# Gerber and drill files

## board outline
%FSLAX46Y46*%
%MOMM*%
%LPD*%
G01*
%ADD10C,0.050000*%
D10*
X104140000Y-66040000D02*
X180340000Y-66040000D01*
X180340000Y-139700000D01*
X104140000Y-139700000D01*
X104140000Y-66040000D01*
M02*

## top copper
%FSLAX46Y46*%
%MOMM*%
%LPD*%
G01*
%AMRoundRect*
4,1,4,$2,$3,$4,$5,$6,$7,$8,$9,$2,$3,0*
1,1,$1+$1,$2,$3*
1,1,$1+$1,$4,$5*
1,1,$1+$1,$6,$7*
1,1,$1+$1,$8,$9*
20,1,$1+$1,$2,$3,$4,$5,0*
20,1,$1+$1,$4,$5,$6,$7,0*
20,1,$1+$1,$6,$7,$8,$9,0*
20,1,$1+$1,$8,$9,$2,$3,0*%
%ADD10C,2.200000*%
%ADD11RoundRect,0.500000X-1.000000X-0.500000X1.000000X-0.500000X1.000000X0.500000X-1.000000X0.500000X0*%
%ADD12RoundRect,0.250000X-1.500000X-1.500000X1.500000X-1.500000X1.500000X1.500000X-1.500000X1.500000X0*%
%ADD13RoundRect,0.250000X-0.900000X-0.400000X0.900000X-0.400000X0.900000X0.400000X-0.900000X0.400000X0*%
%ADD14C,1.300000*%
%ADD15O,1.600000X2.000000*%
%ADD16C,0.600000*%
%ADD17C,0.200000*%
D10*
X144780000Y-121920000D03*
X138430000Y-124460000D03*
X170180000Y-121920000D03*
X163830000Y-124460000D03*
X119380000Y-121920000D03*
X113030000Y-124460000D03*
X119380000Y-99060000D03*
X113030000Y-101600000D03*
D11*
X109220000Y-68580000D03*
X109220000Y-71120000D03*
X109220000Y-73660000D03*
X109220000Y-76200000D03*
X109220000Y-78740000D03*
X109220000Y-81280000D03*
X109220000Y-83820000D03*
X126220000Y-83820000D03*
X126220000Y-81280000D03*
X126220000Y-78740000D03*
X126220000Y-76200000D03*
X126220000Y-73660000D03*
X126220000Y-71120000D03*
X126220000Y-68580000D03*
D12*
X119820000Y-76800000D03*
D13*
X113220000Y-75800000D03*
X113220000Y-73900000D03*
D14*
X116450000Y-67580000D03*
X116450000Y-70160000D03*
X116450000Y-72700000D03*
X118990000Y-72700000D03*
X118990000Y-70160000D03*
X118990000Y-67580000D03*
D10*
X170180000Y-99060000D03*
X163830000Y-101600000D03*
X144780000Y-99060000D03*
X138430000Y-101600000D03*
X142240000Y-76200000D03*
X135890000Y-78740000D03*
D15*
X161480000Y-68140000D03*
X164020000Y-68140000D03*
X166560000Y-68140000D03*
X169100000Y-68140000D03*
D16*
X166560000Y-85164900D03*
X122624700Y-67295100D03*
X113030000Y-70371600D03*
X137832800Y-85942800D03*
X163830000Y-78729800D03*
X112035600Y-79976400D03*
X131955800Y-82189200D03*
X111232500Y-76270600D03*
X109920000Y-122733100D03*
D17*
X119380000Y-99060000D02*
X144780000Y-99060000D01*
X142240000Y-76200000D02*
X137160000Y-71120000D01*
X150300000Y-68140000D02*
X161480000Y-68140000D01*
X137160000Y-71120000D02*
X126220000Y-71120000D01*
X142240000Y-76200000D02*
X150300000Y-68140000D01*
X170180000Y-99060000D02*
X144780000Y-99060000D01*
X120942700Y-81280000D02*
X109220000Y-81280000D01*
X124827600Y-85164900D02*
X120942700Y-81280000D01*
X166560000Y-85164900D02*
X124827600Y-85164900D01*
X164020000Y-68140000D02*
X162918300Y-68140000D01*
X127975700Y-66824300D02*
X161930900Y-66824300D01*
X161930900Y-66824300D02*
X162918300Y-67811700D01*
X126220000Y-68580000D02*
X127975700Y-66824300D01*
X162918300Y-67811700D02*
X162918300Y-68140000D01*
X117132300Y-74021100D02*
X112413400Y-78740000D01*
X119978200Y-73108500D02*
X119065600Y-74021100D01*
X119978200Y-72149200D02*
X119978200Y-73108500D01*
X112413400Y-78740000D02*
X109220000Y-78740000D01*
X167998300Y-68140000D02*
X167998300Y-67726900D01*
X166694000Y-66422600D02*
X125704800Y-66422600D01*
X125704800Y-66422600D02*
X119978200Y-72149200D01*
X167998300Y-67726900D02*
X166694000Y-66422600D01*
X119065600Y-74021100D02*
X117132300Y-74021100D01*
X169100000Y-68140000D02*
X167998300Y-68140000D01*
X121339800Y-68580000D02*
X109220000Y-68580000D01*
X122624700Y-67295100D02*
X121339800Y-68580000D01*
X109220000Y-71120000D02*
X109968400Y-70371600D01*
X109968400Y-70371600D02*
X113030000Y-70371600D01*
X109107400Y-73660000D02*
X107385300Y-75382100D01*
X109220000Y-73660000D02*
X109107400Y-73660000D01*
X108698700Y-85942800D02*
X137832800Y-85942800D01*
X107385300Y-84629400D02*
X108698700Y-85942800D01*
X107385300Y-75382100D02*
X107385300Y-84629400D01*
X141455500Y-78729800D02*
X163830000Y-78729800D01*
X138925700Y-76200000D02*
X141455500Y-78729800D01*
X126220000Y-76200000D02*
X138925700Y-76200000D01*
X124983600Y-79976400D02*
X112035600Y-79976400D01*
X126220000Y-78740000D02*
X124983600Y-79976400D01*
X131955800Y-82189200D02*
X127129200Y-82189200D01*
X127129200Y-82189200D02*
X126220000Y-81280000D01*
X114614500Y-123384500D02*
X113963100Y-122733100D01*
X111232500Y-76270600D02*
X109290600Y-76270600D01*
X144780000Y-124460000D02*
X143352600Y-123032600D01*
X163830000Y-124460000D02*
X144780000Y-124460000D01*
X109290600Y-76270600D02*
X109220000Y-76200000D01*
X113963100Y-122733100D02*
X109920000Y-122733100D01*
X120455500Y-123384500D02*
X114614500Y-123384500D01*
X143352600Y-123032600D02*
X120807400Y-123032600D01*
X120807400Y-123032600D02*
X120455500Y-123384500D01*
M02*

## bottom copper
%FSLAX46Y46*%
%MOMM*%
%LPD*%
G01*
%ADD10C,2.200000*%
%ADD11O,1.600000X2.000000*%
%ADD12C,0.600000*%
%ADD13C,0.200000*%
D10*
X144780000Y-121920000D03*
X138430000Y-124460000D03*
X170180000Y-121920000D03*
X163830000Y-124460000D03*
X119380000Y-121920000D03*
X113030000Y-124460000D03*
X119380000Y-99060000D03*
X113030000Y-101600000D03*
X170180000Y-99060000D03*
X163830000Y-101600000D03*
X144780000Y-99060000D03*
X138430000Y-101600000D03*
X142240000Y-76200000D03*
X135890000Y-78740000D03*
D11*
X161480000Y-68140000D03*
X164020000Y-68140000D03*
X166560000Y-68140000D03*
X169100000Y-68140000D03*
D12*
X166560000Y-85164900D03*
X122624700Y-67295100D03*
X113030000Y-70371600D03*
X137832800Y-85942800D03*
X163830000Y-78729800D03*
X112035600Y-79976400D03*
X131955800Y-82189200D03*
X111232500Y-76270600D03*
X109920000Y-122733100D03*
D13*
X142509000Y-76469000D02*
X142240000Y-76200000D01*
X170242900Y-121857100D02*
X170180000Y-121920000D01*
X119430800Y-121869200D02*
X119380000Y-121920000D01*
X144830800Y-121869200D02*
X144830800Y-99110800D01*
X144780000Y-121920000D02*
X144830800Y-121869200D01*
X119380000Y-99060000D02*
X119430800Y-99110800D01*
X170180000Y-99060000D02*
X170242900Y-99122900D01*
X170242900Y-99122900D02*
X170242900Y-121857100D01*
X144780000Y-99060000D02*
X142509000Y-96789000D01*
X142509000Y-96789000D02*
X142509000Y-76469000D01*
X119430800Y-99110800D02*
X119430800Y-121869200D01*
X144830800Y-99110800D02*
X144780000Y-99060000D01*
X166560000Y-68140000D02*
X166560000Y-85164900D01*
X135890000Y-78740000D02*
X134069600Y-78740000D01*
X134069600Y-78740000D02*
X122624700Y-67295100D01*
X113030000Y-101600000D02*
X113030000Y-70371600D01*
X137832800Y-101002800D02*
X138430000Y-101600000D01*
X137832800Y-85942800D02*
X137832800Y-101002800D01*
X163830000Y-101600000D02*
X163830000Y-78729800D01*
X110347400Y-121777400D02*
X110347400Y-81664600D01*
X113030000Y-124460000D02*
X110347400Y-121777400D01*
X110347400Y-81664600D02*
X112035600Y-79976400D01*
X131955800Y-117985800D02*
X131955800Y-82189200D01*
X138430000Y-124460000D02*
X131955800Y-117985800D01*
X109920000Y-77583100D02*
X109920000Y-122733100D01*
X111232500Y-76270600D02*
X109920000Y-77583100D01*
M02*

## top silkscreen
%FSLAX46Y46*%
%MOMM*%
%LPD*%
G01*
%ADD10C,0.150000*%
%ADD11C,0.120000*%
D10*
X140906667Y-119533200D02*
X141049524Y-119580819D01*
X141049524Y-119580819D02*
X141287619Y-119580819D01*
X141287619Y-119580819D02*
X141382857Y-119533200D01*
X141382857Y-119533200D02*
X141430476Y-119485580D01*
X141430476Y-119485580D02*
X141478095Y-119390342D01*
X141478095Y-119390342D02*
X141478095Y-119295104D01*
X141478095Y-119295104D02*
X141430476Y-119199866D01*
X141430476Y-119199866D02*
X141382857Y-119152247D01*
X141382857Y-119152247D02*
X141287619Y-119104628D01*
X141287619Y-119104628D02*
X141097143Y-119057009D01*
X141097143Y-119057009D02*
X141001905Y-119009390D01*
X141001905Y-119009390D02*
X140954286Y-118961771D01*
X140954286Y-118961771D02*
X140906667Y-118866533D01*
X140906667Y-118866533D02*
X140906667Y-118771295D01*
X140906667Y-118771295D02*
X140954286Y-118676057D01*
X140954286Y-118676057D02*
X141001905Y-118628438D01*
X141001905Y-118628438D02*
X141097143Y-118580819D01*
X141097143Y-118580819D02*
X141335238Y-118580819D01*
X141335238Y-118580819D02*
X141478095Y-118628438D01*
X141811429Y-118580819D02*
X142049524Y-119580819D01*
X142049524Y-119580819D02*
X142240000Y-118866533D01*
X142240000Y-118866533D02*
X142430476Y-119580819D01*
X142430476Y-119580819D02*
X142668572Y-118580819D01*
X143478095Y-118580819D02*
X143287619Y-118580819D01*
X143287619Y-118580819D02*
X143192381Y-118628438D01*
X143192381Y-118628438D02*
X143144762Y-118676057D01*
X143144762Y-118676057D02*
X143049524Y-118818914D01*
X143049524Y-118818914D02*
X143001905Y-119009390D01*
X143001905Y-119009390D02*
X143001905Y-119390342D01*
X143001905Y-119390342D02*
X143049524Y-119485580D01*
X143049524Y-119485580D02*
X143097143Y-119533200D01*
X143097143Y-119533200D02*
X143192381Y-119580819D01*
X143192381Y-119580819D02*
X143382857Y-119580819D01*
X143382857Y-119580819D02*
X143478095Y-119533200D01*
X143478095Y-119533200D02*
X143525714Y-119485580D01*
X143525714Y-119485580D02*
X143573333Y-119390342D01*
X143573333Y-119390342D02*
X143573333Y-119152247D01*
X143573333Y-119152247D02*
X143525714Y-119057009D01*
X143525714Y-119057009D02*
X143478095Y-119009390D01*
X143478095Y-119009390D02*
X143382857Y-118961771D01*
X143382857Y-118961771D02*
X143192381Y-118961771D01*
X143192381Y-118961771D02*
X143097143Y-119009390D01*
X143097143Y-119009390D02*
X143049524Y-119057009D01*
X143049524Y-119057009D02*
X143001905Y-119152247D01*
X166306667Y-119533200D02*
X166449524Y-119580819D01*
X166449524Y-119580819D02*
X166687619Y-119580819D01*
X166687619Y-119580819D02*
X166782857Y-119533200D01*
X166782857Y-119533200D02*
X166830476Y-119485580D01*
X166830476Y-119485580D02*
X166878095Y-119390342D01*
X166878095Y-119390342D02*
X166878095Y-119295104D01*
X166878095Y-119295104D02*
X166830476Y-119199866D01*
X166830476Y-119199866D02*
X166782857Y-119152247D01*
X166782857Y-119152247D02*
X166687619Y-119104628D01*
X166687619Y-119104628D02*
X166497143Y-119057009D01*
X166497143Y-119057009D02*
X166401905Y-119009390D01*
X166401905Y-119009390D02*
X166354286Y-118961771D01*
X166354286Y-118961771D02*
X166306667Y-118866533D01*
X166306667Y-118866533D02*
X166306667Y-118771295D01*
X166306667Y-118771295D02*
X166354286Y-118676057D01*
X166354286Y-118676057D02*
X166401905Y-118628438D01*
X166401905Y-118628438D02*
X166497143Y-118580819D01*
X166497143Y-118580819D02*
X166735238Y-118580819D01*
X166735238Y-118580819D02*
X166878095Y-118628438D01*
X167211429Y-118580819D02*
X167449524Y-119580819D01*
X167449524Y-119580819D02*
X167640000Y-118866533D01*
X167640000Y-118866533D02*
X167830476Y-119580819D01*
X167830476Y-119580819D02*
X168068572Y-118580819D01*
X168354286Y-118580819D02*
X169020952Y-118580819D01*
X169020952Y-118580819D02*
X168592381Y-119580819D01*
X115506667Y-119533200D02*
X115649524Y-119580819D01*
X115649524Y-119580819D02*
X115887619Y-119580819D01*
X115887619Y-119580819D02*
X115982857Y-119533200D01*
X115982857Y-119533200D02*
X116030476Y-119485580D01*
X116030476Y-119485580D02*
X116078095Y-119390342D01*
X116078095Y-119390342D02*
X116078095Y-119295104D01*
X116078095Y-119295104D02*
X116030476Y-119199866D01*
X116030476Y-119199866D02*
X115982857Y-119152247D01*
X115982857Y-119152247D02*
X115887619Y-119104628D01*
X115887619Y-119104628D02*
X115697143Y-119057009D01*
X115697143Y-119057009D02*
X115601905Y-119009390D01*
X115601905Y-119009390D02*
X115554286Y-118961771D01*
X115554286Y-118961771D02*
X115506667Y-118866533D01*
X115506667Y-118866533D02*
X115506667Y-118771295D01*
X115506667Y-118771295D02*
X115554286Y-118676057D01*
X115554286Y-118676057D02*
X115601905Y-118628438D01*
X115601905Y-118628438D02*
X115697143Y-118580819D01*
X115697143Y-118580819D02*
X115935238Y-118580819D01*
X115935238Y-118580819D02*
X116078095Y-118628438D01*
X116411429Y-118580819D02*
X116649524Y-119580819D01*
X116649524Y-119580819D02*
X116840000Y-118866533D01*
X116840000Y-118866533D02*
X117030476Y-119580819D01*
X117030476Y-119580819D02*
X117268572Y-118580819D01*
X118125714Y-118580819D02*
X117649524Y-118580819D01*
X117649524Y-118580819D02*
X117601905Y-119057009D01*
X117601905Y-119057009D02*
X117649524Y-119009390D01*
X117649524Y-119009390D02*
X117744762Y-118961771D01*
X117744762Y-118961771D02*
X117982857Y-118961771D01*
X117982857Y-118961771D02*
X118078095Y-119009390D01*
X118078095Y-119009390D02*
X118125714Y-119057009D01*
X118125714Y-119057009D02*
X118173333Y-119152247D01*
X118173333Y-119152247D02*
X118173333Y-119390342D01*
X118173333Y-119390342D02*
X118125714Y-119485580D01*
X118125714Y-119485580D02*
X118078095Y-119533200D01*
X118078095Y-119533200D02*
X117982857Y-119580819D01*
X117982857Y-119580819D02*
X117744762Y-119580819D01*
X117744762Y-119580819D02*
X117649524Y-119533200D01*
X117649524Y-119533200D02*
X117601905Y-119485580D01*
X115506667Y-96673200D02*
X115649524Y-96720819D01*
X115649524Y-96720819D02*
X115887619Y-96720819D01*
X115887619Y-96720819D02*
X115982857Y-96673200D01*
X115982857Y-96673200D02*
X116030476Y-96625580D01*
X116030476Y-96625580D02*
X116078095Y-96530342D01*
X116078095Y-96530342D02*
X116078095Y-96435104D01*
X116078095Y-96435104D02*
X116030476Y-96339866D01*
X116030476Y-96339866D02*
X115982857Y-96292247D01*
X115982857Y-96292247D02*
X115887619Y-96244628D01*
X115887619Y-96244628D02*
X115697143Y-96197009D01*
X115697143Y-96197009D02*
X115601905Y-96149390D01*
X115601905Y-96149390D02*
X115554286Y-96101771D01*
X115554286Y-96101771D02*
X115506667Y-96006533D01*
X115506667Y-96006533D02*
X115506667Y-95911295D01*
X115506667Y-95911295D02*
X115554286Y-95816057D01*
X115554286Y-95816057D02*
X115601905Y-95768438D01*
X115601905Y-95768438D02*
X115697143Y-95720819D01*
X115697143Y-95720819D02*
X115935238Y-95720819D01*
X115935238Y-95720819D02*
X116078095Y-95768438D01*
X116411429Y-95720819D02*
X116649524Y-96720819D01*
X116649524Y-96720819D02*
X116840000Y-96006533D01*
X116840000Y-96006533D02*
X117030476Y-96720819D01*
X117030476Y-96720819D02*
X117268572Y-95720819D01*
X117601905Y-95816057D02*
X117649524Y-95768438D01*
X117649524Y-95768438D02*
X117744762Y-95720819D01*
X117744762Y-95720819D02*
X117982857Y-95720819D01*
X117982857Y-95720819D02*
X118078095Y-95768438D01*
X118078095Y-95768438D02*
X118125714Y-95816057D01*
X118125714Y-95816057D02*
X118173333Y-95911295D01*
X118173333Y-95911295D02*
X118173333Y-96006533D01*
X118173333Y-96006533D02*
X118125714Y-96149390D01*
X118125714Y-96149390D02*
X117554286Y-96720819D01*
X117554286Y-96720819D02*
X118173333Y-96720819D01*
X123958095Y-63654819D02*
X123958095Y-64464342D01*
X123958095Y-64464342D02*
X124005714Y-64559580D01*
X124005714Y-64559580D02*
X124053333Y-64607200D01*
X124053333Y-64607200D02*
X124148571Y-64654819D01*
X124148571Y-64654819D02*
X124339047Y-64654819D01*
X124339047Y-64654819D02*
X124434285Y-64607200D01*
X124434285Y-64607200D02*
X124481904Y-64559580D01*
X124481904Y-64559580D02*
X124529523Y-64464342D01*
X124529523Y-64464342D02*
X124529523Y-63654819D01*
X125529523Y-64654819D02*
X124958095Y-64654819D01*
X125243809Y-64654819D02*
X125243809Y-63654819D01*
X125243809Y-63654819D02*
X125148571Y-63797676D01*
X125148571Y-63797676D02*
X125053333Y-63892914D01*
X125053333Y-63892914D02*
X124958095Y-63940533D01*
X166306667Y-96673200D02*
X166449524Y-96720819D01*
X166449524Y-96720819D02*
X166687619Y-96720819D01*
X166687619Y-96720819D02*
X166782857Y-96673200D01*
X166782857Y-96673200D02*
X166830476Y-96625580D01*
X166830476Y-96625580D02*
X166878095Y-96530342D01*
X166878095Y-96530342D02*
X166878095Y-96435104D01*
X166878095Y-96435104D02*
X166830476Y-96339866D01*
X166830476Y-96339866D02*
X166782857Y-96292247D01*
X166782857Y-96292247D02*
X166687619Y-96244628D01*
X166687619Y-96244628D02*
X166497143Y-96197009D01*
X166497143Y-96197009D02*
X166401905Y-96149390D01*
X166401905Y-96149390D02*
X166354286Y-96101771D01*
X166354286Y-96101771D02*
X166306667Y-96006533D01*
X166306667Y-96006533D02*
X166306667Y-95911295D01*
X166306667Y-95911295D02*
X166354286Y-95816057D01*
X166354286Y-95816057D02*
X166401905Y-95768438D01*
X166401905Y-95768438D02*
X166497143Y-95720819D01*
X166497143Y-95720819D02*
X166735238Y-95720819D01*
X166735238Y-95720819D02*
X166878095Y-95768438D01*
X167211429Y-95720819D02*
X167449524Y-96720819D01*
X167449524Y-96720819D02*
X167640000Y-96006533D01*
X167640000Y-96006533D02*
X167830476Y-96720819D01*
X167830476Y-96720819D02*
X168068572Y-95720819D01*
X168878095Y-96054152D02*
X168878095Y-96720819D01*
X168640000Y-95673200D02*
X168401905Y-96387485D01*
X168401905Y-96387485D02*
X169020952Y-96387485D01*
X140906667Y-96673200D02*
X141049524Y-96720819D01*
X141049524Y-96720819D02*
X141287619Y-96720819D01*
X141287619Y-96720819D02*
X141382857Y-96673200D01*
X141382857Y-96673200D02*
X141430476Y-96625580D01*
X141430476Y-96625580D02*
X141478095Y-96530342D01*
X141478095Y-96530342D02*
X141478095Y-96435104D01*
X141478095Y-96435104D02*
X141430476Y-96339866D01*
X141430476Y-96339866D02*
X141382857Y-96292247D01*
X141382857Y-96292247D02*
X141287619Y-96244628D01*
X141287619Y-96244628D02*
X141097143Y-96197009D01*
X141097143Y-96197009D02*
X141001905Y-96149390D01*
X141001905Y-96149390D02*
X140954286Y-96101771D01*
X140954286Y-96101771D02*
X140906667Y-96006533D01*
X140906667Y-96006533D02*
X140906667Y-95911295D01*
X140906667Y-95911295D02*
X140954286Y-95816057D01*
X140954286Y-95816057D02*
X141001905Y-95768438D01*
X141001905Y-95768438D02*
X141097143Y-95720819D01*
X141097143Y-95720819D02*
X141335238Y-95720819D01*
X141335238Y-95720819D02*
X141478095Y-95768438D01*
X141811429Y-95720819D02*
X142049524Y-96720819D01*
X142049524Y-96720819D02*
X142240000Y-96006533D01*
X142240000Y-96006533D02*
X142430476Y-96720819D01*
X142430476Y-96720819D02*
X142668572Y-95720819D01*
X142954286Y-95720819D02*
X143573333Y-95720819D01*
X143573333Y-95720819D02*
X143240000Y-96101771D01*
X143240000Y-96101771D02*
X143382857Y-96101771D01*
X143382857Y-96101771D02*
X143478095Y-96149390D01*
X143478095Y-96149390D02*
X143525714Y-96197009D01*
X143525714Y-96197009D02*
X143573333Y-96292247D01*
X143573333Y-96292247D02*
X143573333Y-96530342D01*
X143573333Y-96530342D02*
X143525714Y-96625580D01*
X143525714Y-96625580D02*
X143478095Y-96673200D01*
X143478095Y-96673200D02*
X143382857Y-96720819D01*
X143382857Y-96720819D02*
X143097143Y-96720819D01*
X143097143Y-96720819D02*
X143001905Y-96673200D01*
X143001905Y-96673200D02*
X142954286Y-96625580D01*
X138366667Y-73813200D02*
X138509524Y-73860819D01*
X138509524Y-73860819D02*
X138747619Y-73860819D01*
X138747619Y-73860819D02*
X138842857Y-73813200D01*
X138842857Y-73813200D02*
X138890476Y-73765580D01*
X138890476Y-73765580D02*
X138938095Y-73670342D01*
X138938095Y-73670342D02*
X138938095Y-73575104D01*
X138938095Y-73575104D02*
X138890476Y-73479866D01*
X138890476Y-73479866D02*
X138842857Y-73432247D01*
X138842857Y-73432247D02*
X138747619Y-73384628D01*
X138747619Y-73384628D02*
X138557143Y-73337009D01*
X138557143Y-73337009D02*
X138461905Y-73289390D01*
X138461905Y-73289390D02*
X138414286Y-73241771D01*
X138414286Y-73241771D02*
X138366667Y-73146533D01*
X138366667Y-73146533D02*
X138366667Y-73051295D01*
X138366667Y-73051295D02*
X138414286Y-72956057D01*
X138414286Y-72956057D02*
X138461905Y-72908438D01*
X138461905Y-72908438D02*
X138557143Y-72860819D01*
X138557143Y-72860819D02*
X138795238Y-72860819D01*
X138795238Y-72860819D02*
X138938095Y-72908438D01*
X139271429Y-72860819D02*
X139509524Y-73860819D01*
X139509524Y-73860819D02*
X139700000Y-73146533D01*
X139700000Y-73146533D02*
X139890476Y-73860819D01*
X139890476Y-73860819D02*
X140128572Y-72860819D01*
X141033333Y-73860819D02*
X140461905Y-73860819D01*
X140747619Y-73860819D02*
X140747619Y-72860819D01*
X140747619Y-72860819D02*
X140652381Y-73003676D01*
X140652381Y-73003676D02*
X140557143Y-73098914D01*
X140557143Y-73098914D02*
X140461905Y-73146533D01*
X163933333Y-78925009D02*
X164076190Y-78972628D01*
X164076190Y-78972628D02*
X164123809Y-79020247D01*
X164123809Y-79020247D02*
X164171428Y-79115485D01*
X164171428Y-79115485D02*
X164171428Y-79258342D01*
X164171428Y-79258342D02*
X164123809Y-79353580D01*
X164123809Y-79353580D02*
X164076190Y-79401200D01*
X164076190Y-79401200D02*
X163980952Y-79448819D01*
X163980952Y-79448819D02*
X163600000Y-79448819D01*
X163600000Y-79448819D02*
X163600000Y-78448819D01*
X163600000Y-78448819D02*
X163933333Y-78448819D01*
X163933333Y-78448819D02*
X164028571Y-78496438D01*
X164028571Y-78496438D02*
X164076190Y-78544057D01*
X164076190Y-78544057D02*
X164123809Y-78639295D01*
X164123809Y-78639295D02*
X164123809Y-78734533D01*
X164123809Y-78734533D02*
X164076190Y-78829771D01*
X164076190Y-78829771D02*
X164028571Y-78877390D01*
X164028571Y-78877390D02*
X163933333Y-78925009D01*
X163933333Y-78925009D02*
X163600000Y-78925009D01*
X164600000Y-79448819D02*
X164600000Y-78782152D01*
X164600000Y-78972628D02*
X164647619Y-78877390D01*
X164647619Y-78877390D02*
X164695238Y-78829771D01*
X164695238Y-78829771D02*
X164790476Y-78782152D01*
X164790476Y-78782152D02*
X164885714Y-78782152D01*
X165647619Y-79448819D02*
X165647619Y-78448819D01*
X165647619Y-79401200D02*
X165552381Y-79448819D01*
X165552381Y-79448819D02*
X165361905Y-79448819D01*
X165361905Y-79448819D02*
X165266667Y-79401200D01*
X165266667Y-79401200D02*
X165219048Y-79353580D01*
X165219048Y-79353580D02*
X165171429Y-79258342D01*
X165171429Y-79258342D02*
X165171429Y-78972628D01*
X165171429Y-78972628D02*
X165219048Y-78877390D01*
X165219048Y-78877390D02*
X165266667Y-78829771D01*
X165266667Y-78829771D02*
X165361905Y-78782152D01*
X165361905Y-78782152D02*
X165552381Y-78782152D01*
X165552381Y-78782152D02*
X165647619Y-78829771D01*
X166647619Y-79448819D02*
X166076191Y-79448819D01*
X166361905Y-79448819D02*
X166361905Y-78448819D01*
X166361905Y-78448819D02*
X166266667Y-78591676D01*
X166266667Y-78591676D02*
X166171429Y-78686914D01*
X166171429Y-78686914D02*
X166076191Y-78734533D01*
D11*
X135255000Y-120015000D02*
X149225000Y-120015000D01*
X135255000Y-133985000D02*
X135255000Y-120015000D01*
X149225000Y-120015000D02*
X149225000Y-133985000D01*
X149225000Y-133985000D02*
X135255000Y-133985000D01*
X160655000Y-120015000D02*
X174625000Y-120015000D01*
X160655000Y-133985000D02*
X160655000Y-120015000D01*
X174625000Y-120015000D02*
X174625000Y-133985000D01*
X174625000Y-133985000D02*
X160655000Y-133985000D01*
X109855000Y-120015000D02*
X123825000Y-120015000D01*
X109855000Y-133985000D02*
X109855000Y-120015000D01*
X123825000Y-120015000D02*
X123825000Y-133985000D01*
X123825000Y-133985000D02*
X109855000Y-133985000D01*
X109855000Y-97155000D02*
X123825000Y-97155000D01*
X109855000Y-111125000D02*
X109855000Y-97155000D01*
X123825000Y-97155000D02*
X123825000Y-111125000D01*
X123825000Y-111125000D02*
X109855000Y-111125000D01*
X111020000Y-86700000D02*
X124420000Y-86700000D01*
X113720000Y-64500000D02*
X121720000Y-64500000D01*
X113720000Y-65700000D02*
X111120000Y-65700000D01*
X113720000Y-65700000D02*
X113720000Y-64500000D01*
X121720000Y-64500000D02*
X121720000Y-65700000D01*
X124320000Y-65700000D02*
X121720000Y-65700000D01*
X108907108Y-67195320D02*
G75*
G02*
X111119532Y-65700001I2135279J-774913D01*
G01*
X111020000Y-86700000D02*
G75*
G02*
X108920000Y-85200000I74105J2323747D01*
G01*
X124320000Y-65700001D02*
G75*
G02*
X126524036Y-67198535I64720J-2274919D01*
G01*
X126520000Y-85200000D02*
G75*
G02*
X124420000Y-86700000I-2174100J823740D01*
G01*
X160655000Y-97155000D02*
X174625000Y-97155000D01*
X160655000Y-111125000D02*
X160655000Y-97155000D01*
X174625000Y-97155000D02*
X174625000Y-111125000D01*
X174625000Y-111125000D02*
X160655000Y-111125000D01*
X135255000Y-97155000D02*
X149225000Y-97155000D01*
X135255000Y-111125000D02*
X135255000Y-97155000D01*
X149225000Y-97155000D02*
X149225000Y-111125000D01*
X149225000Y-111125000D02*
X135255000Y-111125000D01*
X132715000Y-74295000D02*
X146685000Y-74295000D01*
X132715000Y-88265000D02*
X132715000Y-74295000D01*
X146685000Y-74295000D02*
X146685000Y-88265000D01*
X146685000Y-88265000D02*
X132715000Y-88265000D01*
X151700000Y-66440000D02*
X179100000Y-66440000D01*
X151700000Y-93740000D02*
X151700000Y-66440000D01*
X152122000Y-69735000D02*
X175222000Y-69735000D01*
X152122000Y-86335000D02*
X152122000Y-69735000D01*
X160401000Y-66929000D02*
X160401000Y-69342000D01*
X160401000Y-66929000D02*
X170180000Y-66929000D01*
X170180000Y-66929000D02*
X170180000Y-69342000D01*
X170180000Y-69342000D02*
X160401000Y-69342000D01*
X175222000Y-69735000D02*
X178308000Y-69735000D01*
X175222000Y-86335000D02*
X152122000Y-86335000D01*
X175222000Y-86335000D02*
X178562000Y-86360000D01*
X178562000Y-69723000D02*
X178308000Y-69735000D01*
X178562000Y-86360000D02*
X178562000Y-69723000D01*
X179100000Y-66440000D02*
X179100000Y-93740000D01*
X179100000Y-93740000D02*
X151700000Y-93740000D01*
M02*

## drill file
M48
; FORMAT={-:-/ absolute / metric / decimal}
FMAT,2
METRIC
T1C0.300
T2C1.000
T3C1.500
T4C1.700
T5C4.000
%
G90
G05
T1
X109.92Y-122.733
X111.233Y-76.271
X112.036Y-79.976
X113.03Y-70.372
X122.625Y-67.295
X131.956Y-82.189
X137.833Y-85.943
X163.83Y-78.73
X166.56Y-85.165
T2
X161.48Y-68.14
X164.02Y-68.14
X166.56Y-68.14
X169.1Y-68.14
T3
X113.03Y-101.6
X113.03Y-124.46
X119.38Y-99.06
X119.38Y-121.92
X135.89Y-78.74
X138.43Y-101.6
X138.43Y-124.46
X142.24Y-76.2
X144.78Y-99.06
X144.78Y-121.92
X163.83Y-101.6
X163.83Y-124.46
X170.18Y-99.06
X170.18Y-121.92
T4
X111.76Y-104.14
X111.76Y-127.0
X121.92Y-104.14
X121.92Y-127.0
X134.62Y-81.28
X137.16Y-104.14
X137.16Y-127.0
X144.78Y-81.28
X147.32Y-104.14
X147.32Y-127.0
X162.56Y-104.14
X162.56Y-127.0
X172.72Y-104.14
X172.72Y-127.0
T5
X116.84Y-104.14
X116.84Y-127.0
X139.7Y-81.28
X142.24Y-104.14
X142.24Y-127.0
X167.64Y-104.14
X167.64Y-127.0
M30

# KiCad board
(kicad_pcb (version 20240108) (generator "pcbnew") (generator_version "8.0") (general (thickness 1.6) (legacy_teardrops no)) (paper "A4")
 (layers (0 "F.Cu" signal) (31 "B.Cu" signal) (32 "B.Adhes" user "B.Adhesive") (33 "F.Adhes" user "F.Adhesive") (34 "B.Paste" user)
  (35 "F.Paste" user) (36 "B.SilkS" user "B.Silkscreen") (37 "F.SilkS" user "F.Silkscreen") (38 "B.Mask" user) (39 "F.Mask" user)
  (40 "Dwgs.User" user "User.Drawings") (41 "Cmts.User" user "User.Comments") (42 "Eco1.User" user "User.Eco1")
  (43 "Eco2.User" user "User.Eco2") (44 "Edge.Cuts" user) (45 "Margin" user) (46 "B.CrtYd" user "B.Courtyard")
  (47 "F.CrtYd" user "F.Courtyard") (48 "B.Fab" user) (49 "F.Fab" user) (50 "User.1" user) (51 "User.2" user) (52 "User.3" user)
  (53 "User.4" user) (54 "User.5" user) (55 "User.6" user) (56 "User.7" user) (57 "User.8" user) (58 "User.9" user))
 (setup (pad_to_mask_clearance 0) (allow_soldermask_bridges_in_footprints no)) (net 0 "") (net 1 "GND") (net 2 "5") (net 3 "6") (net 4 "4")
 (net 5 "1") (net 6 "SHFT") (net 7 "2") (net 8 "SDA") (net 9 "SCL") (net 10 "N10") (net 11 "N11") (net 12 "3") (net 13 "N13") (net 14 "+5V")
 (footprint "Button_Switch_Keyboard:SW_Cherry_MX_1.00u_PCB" (layer "F.Cu") (at 144.78 121.92)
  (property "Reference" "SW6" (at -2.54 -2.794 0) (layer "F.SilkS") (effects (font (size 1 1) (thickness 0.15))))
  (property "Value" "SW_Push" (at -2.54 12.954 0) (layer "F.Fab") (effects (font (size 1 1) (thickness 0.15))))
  (fp_line (start -9.525 -1.905) (end 4.445 -1.905) (stroke (width 0.12) (type solid)) (layer "F.SilkS"))
  (fp_line (start -9.525 12.065) (end -9.525 -1.905) (stroke (width 0.12) (type solid)) (layer "F.SilkS"))
  (fp_line (start 4.445 -1.905) (end 4.445 12.065) (stroke (width 0.12) (type solid)) (layer "F.SilkS"))
  (fp_line (start 4.445 12.065) (end -9.525 12.065) (stroke (width 0.12) (type solid)) (layer "F.SilkS"))
  (pad "" np_thru_hole circle (at -7.62 5.08) (size 1.7 1.7) (drill 1.7) (layers "*.Cu" "*.Mask"))
  (pad "" np_thru_hole circle (at -2.54 5.08) (size 4 4) (drill 4) (layers "*.Cu" "*.Mask"))
  (pad "" np_thru_hole circle (at 2.54 5.08) (size 1.7 1.7) (drill 1.7) (layers "*.Cu" "*.Mask"))
  (pad "1" thru_hole circle (at 0 0) (size 2.2 2.2) (drill 1.5) (layers "*.Cu" "*.Mask") (remove_unused_layers no) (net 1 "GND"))
  (pad "2" thru_hole circle (at -6.35 2.54) (size 2.2 2.2) (drill 1.5) (layers "*.Cu" "*.Mask") (remove_unused_layers no) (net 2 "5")))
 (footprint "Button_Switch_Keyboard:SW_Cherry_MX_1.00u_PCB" (layer "F.Cu") (at 170.18 121.92)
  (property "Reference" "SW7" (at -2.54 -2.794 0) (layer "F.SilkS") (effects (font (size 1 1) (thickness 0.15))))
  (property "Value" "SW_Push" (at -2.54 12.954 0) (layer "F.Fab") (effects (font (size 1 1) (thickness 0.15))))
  (fp_line (start -9.525 -1.905) (end 4.445 -1.905) (stroke (width 0.12) (type solid)) (layer "F.SilkS"))
  (fp_line (start -9.525 12.065) (end -9.525 -1.905) (stroke (width 0.12) (type solid)) (layer "F.SilkS"))
  (fp_line (start 4.445 -1.905) (end 4.445 12.065) (stroke (width 0.12) (type solid)) (layer "F.SilkS"))
  (fp_line (start 4.445 12.065) (end -9.525 12.065) (stroke (width 0.12) (type solid)) (layer "F.SilkS"))
  (pad "" np_thru_hole circle (at -7.62 5.08) (size 1.7 1.7) (drill 1.7) (layers "*.Cu" "*.Mask"))
  (pad "" np_thru_hole circle (at -2.54 5.08) (size 4 4) (drill 4) (layers "*.Cu" "*.Mask"))
  (pad "" np_thru_hole circle (at 2.54 5.08) (size 1.7 1.7) (drill 1.7) (layers "*.Cu" "*.Mask"))
  (pad "1" thru_hole circle (at 0 0) (size 2.2 2.2) (drill 1.5) (layers "*.Cu" "*.Mask") (remove_unused_layers no) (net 1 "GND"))
  (pad "2" thru_hole circle (at -6.35 2.54) (size 2.2 2.2) (drill 1.5) (layers "*.Cu" "*.Mask") (remove_unused_layers no) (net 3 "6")))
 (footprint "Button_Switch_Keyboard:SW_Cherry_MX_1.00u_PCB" (layer "F.Cu") (at 119.38 121.92)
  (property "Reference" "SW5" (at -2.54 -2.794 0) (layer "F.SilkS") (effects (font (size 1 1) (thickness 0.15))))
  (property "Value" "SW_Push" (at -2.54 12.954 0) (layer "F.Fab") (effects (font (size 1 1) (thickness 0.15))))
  (fp_line (start -9.525 -1.905) (end 4.445 -1.905) (stroke (width 0.12) (type solid)) (layer "F.SilkS"))
  (fp_line (start -9.525 12.065) (end -9.525 -1.905) (stroke (width 0.12) (type solid)) (layer "F.SilkS"))
  (fp_line (start 4.445 -1.905) (end 4.445 12.065) (stroke (width 0.12) (type solid)) (layer "F.SilkS"))
  (fp_line (start 4.445 12.065) (end -9.525 12.065) (stroke (width 0.12) (type solid)) (layer "F.SilkS"))
  (pad "" np_thru_hole circle (at -7.62 5.08) (size 1.7 1.7) (drill 1.7) (layers "*.Cu" "*.Mask"))
  (pad "" np_thru_hole circle (at -2.54 5.08) (size 4 4) (drill 4) (layers "*.Cu" "*.Mask"))
  (pad "" np_thru_hole circle (at 2.54 5.08) (size 1.7 1.7) (drill 1.7) (layers "*.Cu" "*.Mask"))
  (pad "1" thru_hole circle (at 0 0) (size 2.2 2.2) (drill 1.5) (layers "*.Cu" "*.Mask") (remove_unused_layers no) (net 1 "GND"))
  (pad "2" thru_hole circle (at -6.35 2.54) (size 2.2 2.2) (drill 1.5) (layers "*.Cu" "*.Mask") (remove_unused_layers no) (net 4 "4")))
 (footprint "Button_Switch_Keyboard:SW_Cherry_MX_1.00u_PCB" (layer "F.Cu") (at 119.38 99.06)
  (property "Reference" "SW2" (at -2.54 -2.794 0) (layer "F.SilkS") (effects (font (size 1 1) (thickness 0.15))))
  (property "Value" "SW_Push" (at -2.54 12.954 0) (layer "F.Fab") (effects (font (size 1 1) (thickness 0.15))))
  (fp_line (start -9.525 -1.905) (end 4.445 -1.905) (stroke (width 0.12) (type solid)) (layer "F.SilkS"))
  (fp_line (start -9.525 12.065) (end -9.525 -1.905) (stroke (width 0.12) (type solid)) (layer "F.SilkS"))
  (fp_line (start 4.445 -1.905) (end 4.445 12.065) (stroke (width 0.12) (type solid)) (layer "F.SilkS"))
  (fp_line (start 4.445 12.065) (end -9.525 12.065) (stroke (width 0.12) (type solid)) (layer "F.SilkS"))
  (pad "" np_thru_hole circle (at -7.62 5.08) (size 1.7 1.7) (drill 1.7) (layers "*.Cu" "*.Mask"))
  (pad "" np_thru_hole circle (at -2.54 5.08) (size 4 4) (drill 4) (layers "*.Cu" "*.Mask"))
  (pad "" np_thru_hole circle (at 2.54 5.08) (size 1.7 1.7) (drill 1.7) (layers "*.Cu" "*.Mask"))
  (pad "1" thru_hole circle (at 0 0) (size 2.2 2.2) (drill 1.5) (layers "*.Cu" "*.Mask") (remove_unused_layers no) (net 1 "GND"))
  (pad "2" thru_hole circle (at -6.35 2.54) (size 2.2 2.2) (drill 1.5) (layers "*.Cu" "*.Mask") (remove_unused_layers no) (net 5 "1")))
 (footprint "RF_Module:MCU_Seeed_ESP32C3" (layer "F.Cu") (at 117.72 76.2)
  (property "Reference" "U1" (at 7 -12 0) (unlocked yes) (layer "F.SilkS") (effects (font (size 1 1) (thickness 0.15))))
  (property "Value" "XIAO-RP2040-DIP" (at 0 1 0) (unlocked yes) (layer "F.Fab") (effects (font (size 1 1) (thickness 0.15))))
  (fp_line (start -6.7 10.5) (end 6.7 10.5) (stroke (width 0.12) (type default)) (layer "F.SilkS"))
  (fp_line (start -4 -11.7) (end 4 -11.7) (stroke (width 0.12) (type default)) (layer "F.SilkS"))
  (fp_line (start -4 -10.5) (end -6.6 -10.5) (stroke (width 0.12) (type default)) (layer "F.SilkS"))
  (fp_line (start -4 -10.5) (end -4 -11.7) (stroke (width 0.12) (type default)) (layer "F.SilkS"))
  (fp_line (start 4 -11.7) (end 4 -10.5) (stroke (width 0.12) (type default)) (layer "F.SilkS"))
  (fp_line (start 6.6 -10.5) (end 4 -10.5) (stroke (width 0.12) (type default)) (layer "F.SilkS"))
  (fp_arc (start -8.812892 -9.00468) (mid -7.949609 -10.111769) (end -6.600468 -10.499999) (stroke (width 0.12) (type default))
   (layer "F.SilkS"))
  (fp_arc (start -6.7 10.5) (mid -7.977232 10.068125) (end -8.8 9) (stroke (width 0.12) (type default)) (layer "F.SilkS"))
  (fp_arc (start 6.6 -10.499999) (mid 7.944323 -10.107114) (end 8.804034 -9.001464) (stroke (width 0.12) (type default)) (layer "F.SilkS"))
  (fp_arc (start 8.8 9) (mid 7.977232 10.068126) (end 6.7 10.5) (stroke (width 0.12) (type default)) (layer "F.SilkS"))
  (pad "" smd roundrect (at 1.1 -0.4) (size 1.5 1.5) (layers "F.Paste") (roundrect_rratio 0.1666666667))
  (pad "" smd roundrect (at 1.1 1.6) (size 1.5 1.5) (layers "F.Paste") (roundrect_rratio 0.1666666667))
  (pad "" smd roundrect (at 3.1 -0.4) (size 1.5 1.5) (layers "F.Paste") (roundrect_rratio 0.1666666667))
  (pad "" smd roundrect (at 3.1 1.6) (size 1.5 1.5) (layers "F.Paste") (roundrect_rratio 0.1666666667))
  (pad "1" smd roundrect (at -8.5 -7.62) (size 3 2) (layers "F.Cu" "F.Paste" "F.Mask") (roundrect_rratio 0.25) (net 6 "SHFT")
   (thermal_bridge_angle 45))
  (pad "2" smd roundrect (at -8.5 -5.08) (size 3 2) (layers "F.Cu" "F.Paste" "F.Mask") (roundrect_rratio 0.25) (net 5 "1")
   (thermal_bridge_angle 45))
  (pad "3" smd roundrect (at -8.5 -2.54) (size 3 2) (layers "F.Cu" "F.Paste" "F.Mask") (roundrect_rratio 0.25) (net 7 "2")
   (thermal_bridge_angle 45))
  (pad "4" smd roundrect (at -8.5 0) (size 3 2) (layers "F.Cu" "F.Paste" "F.Mask") (roundrect_rratio 0.25) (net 3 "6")
   (thermal_bridge_angle 45))
  (pad "5" smd roundrect (at -8.5 2.54) (size 3 2) (layers "F.Cu" "F.Paste" "F.Mask") (roundrect_rratio 0.25) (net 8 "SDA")
   (thermal_bridge_angle 45))
  (pad "6" smd roundrect (at -8.5 5.08) (size 3 2) (layers "F.Cu" "F.Paste" "F.Mask") (roundrect_rratio 0.25) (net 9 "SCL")
   (thermal_bridge_angle 45))
  (pad "7" smd roundrect (at -8.5 7.62) (size 3 2) (layers "F.Cu" "F.Paste" "F.Mask") (roundrect_rratio 0.25) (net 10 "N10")
   (thermal_bridge_angle 45))
  (pad "8" smd roundrect (at 8.5 7.62) (size 3 2) (layers "F.Cu" "F.Paste" "F.Mask") (roundrect_rratio 0.25) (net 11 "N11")
   (thermal_bridge_angle 45))
  (pad "9" smd roundrect (at 8.5 5.08) (size 3 2) (layers "F.Cu" "F.Paste" "F.Mask") (roundrect_rratio 0.25) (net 2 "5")
   (thermal_bridge_angle 45))
  (pad "10" smd roundrect (at 8.5 2.54) (size 3 2) (layers "F.Cu" "F.Paste" "F.Mask") (roundrect_rratio 0.25) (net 4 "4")
   (thermal_bridge_angle 45))
  (pad "11" smd roundrect (at 8.5 0) (size 3 2) (layers "F.Cu" "F.Paste" "F.Mask") (roundrect_rratio 0.25) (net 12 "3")
   (thermal_bridge_angle 45))
  (pad "12" smd roundrect (at 8.5 -2.54) (size 3 2) (layers "F.Cu" "F.Paste" "F.Mask") (roundrect_rratio 0.25) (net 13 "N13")
   (thermal_bridge_angle 45))
  (pad "13" smd roundrect (at 8.5 -5.08) (size 3 2) (layers "F.Cu" "F.Paste" "F.Mask") (roundrect_rratio 0.25) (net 1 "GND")
   (thermal_bridge_angle 45))
  (pad "14" smd roundrect (at 8.5 -7.62) (size 3 2) (layers "F.Cu" "F.Paste" "F.Mask") (roundrect_rratio 0.25) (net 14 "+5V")
   (thermal_bridge_angle 45))
  (pad "15" smd roundrect (at 2.1 0.6) (size 3.5 3.5) (layers "F.Cu" "F.Mask") (roundrect_rratio 0.07142857143))
  (pad "16" smd roundrect (at -4.5 -0.4) (size 2.3 1.3) (layers "F.Cu" "F.Paste" "F.Mask") (roundrect_rratio 0.1923076923))
  (pad "17" smd roundrect (at -4.5 -2.3) (size 2.3 1.3) (layers "F.Cu" "F.Paste" "F.Mask") (roundrect_rratio 0.1923076923))
  (pad "18" smd circle (at -1.27 -8.62) (size 1.3 1.3) (layers "F.Cu" "F.Paste" "F.Mask"))
  (pad "19" smd circle (at -1.27 -6.04) (size 1.3 1.3) (layers "F.Cu" "F.Paste" "F.Mask"))
  (pad "20" smd circle (at -1.27 -3.5) (size 1.3 1.3) (layers "F.Cu" "F.Paste" "F.Mask"))
  (pad "21" smd circle (at 1.27 -3.5) (size 1.3 1.3) (layers "F.Cu" "F.Paste" "F.Mask"))
  (pad "22" smd circle (at 1.27 -6.04) (size 1.3 1.3) (layers "F.Cu" "F.Paste" "F.Mask"))
  (pad "23" smd circle (at 1.27 -8.62) (size 1.3 1.3) (layers "F.Cu" "F.Paste" "F.Mask")))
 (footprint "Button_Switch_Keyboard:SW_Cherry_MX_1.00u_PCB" (layer "F.Cu") (at 170.18 99.06)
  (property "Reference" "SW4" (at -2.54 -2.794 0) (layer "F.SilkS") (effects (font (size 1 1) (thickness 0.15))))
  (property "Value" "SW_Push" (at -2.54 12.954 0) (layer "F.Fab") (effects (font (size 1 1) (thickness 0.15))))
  (fp_line (start -9.525 -1.905) (end 4.445 -1.905) (stroke (width 0.12) (type solid)) (layer "F.SilkS"))
  (fp_line (start -9.525 12.065) (end -9.525 -1.905) (stroke (width 0.12) (type solid)) (layer "F.SilkS"))
  (fp_line (start 4.445 -1.905) (end 4.445 12.065) (stroke (width 0.12) (type solid)) (layer "F.SilkS"))
  (fp_line (start 4.445 12.065) (end -9.525 12.065) (stroke (width 0.12) (type solid)) (layer "F.SilkS"))
  (pad "" np_thru_hole circle (at -7.62 5.08) (size 1.7 1.7) (drill 1.7) (layers "*.Cu" "*.Mask"))
  (pad "" np_thru_hole circle (at -2.54 5.08) (size 4 4) (drill 4) (layers "*.Cu" "*.Mask"))
  (pad "" np_thru_hole circle (at 2.54 5.08) (size 1.7 1.7) (drill 1.7) (layers "*.Cu" "*.Mask"))
  (pad "1" thru_hole circle (at 0 0) (size 2.2 2.2) (drill 1.5) (layers "*.Cu" "*.Mask") (remove_unused_layers no) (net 1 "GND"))
  (pad "2" thru_hole circle (at -6.35 2.54) (size 2.2 2.2) (drill 1.5) (layers "*.Cu" "*.Mask") (remove_unused_layers no) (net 12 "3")))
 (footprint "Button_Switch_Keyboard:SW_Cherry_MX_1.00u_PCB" (layer "F.Cu") (at 144.78 99.06)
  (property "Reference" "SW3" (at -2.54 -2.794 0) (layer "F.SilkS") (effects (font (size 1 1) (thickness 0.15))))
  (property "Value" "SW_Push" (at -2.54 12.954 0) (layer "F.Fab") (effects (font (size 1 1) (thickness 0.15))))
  (fp_line (start -9.525 -1.905) (end 4.445 -1.905) (stroke (width 0.12) (type solid)) (layer "F.SilkS"))
  (fp_line (start -9.525 12.065) (end -9.525 -1.905) (stroke (width 0.12) (type solid)) (layer "F.SilkS"))
  (fp_line (start 4.445 -1.905) (end 4.445 12.065) (stroke (width 0.12) (type solid)) (layer "F.SilkS"))
  (fp_line (start 4.445 12.065) (end -9.525 12.065) (stroke (width 0.12) (type solid)) (layer "F.SilkS"))
  (pad "" np_thru_hole circle (at -7.62 5.08) (size 1.7 1.7) (drill 1.7) (layers "*.Cu" "*.Mask"))
  (pad "" np_thru_hole circle (at -2.54 5.08) (size 4 4) (drill 4) (layers "*.Cu" "*.Mask"))
  (pad "" np_thru_hole circle (at 2.54 5.08) (size 1.7 1.7) (drill 1.7) (layers "*.Cu" "*.Mask"))
  (pad "1" thru_hole circle (at 0 0) (size 2.2 2.2) (drill 1.5) (layers "*.Cu" "*.Mask") (remove_unused_layers no) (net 1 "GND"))
  (pad "2" thru_hole circle (at -6.35 2.54) (size 2.2 2.2) (drill 1.5) (layers "*.Cu" "*.Mask") (remove_unused_layers no) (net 7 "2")))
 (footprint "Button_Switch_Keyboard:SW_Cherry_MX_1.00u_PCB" (layer "F.Cu") (at 142.24 76.2)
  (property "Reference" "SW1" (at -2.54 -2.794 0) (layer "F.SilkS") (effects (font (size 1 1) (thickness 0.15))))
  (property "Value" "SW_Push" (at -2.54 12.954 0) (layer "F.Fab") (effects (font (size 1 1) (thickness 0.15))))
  (fp_line (start -9.525 -1.905) (end 4.445 -1.905) (stroke (width 0.12) (type solid)) (layer "F.SilkS"))
  (fp_line (start -9.525 12.065) (end -9.525 -1.905) (stroke (width 0.12) (type solid)) (layer "F.SilkS"))
  (fp_line (start 4.445 -1.905) (end 4.445 12.065) (stroke (width 0.12) (type solid)) (layer "F.SilkS"))
  (fp_line (start 4.445 12.065) (end -9.525 12.065) (stroke (width 0.12) (type solid)) (layer "F.SilkS"))
  (pad "" np_thru_hole circle (at -7.62 5.08) (size 1.7 1.7) (drill 1.7) (layers "*.Cu" "*.Mask"))
  (pad "" np_thru_hole circle (at -2.54 5.08) (size 4 4) (drill 4) (layers "*.Cu" "*.Mask"))
  (pad "" np_thru_hole circle (at 2.54 5.08) (size 1.7 1.7) (drill 1.7) (layers "*.Cu" "*.Mask"))
  (pad "1" thru_hole circle (at 0 0) (size 2.2 2.2) (drill 1.5) (layers "*.Cu" "*.Mask") (remove_unused_layers no) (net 1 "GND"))
  (pad "2" thru_hole circle (at -6.35 2.54) (size 2.2 2.2) (drill 1.5) (layers "*.Cu" "*.Mask") (remove_unused_layers no) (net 6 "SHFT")))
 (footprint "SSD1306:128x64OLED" (layer "F.Cu") (at 165.1 78.74)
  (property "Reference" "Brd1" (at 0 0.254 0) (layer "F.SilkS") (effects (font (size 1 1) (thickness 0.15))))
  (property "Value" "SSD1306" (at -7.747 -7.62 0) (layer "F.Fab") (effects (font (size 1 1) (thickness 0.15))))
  (fp_line (start -13.4 -12.3) (end 14 -12.3) (stroke (width 0.12) (type solid)) (layer "F.SilkS"))
  (fp_line (start -13.4 15) (end -13.4 -12.3) (stroke (width 0.12) (type solid)) (layer "F.SilkS"))
  (fp_line (start -12.978 -9.005) (end 10.122 -9.005) (stroke (width 0.12) (type solid)) (layer "F.SilkS"))
  (fp_line (start -12.978 7.595) (end -12.978 -9.005) (stroke (width 0.12) (type solid)) (layer "F.SilkS"))
  (fp_line (start -4.699 -11.811) (end -4.699 -9.398) (stroke (width 0.12) (type solid)) (layer "F.SilkS"))
  (fp_line (start -4.699 -11.811) (end 5.08 -11.811) (stroke (width 0.12) (type solid)) (layer "F.SilkS"))
  (fp_line (start 5.08 -11.811) (end 5.08 -9.398) (stroke (width 0.12) (type solid)) (layer "F.SilkS"))
  (fp_line (start 5.08 -9.398) (end -4.699 -9.398) (stroke (width 0.12) (type solid)) (layer "F.SilkS"))
  (fp_line (start 10.122 -9.005) (end 13.208 -9.005) (stroke (width 0.12) (type solid)) (layer "F.SilkS"))
  (fp_line (start 10.122 7.595) (end -12.978 7.595) (stroke (width 0.12) (type solid)) (layer "F.SilkS"))
  (fp_line (start 10.122 7.595) (end 13.462 7.62) (stroke (width 0.12) (type solid)) (layer "F.SilkS"))
  (fp_line (start 13.462 -9.017) (end 13.208 -9.005) (stroke (width 0.12) (type solid)) (layer "F.SilkS"))
  (fp_line (start 13.462 7.62) (end 13.462 -9.017) (stroke (width 0.12) (type solid)) (layer "F.SilkS"))
  (fp_line (start 14 -12.3) (end 14 15) (stroke (width 0.12) (type solid)) (layer "F.SilkS"))
  (fp_line (start 14 15) (end -13.4 15) (stroke (width 0.12) (type solid)) (layer "F.SilkS"))
  (pad "1" thru_hole oval (at -3.62 -10.6 90) (size 2 1.6) (drill 1) (layers "*.Cu" "*.Mask") (remove_unused_layers no) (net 1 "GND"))
  (pad "2" thru_hole oval (at -1.08 -10.6 90) (size 2 1.6) (drill 1) (layers "*.Cu" "*.Mask") (remove_unused_layers no) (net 14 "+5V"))
  (pad "3" thru_hole oval (at 1.46 -10.6 90) (size 2 1.6) (drill 1) (layers "*.Cu" "*.Mask") (remove_unused_layers no) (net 9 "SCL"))
  (pad "4" thru_hole oval (at 4 -10.6 90) (size 2 1.6) (drill 1) (layers "*.Cu" "*.Mask") (remove_unused_layers no) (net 8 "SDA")))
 (gr_rect (start 104.14 66.04) (end 180.34 139.7) (stroke (width 0.05) (type default)) (fill none) (layer "Edge.Cuts"))
 (segment (start 119.38 99.06) (end 144.78 99.06) (width 0.2) (layer "F.Cu") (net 1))
 (segment (start 142.24 76.2) (end 137.16 71.12) (width 0.2) (layer "F.Cu") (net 1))
 (segment (start 150.3 68.14) (end 161.48 68.14) (width 0.2) (layer "F.Cu") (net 1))
 (segment (start 137.16 71.12) (end 126.22 71.12) (width 0.2) (layer "F.Cu") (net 1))
 (segment (start 142.24 76.2) (end 150.3 68.14) (width 0.2) (layer "F.Cu") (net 1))
 (segment (start 170.18 99.06) (end 144.78 99.06) (width 0.2) (layer "F.Cu") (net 1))
 (segment (start 142.509 76.469) (end 142.24 76.2) (width 0.2) (layer "B.Cu") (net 1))
 (segment (start 170.2429 121.8571) (end 170.18 121.92) (width 0.2) (layer "B.Cu") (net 1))
 (segment (start 119.4308 121.8692) (end 119.38 121.92) (width 0.2) (layer "B.Cu") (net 1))
 (segment (start 144.8308 121.8692) (end 144.8308 99.1108) (width 0.2) (layer "B.Cu") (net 1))
 (segment (start 144.78 121.92) (end 144.8308 121.8692) (width 0.2) (layer "B.Cu") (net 1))
 (segment (start 119.38 99.06) (end 119.4308 99.1108) (width 0.2) (layer "B.Cu") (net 1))
 (segment (start 170.18 99.06) (end 170.2429 99.1229) (width 0.2) (layer "B.Cu") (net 1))
 (segment (start 170.2429 99.1229) (end 170.2429 121.8571) (width 0.2) (layer "B.Cu") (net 1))
 (segment (start 144.78 99.06) (end 142.509 96.789) (width 0.2) (layer "B.Cu") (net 1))
 (segment (start 142.509 96.789) (end 142.509 76.469) (width 0.2) (layer "B.Cu") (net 1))
 (segment (start 119.4308 99.1108) (end 119.4308 121.8692) (width 0.2) (layer "B.Cu") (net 1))
 (segment (start 144.8308 99.1108) (end 144.78 99.06) (width 0.2) (layer "B.Cu") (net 1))
 (segment (start 120.9427 81.28) (end 109.22 81.28) (width 0.2) (layer "F.Cu") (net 9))
 (segment (start 124.8276 85.1649) (end 120.9427 81.28) (width 0.2) (layer "F.Cu") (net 9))
 (segment (start 166.56 85.1649) (end 124.8276 85.1649) (width 0.2) (layer "F.Cu") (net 9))
 (via (at 166.56 85.1649) (size 0.6) (drill 0.3) (layers "F.Cu" "B.Cu") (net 9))
 (segment (start 166.56 68.14) (end 166.56 85.1649) (width 0.2) (layer "B.Cu") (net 9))
 (segment (start 164.02 68.14) (end 162.9183 68.14) (width 0.2) (layer "F.Cu") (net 14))
 (segment (start 127.9757 66.8243) (end 161.9309 66.8243) (width 0.2) (layer "F.Cu") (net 14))
 (segment (start 161.9309 66.8243) (end 162.9183 67.8117) (width 0.2) (layer "F.Cu") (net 14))
 (segment (start 126.22 68.58) (end 127.9757 66.8243) (width 0.2) (layer "F.Cu") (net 14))
 (segment (start 162.9183 67.8117) (end 162.9183 68.14) (width 0.2) (layer "F.Cu") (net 14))
 (segment (start 117.1323 74.0211) (end 112.4134 78.74) (width 0.2) (layer "F.Cu") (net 8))
 (segment (start 119.9782 73.1085) (end 119.0656 74.0211) (width 0.2) (layer "F.Cu") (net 8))
 (segment (start 119.9782 72.1492) (end 119.9782 73.1085) (width 0.2) (layer "F.Cu") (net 8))
 (segment (start 112.4134 78.74) (end 109.22 78.74) (width 0.2) (layer "F.Cu") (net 8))
 (segment (start 167.9983 68.14) (end 167.9983 67.7269) (width 0.2) (layer "F.Cu") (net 8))
 (segment (start 166.694 66.4226) (end 125.7048 66.4226) (width 0.2) (layer "F.Cu") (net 8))
 (segment (start 125.7048 66.4226) (end 119.9782 72.1492) (width 0.2) (layer "F.Cu") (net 8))
 (segment (start 167.9983 67.7269) (end 166.694 66.4226) (width 0.2) (layer "F.Cu") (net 8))
 (segment (start 119.0656 74.0211) (end 117.1323 74.0211) (width 0.2) (layer "F.Cu") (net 8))
 (segment (start 169.1 68.14) (end 167.9983 68.14) (width 0.2) (layer "F.Cu") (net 8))
 (segment (start 121.3398 68.58) (end 109.22 68.58) (width 0.2) (layer "F.Cu") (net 6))
 (segment (start 122.6247 67.2951) (end 121.3398 68.58) (width 0.2) (layer "F.Cu") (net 6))
 (via (at 122.6247 67.2951) (size 0.6) (drill 0.3) (layers "F.Cu" "B.Cu") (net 6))
 (segment (start 135.89 78.74) (end 134.0696 78.74) (width 0.2) (layer "B.Cu") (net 6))
 (segment (start 134.0696 78.74) (end 122.6247 67.2951) (width 0.2) (layer "B.Cu") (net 6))
 (segment (start 109.22 71.12) (end 109.9684 70.3716) (width 0.2) (layer "F.Cu") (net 5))
 (segment (start 109.9684 70.3716) (end 113.03 70.3716) (width 0.2) (layer "F.Cu") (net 5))
 (via (at 113.03 70.3716) (size 0.6) (drill 0.3) (layers "F.Cu" "B.Cu") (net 5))
 (segment (start 113.03 101.6) (end 113.03 70.3716) (width 0.2) (layer "B.Cu") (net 5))
 (segment (start 109.1074 73.66) (end 107.3853 75.3821) (width 0.2) (layer "F.Cu") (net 7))
 (segment (start 109.22 73.66) (end 109.1074 73.66) (width 0.2) (layer "F.Cu") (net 7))
 (segment (start 108.6987 85.9428) (end 137.8328 85.9428) (width 0.2) (layer "F.Cu") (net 7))
 (segment (start 107.3853 84.6294) (end 108.6987 85.9428) (width 0.2) (layer "F.Cu") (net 7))
 (segment (start 107.3853 75.3821) (end 107.3853 84.6294) (width 0.2) (layer "F.Cu") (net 7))
 (via (at 137.8328 85.9428) (size 0.6) (drill 0.3) (layers "F.Cu" "B.Cu") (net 7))
 (segment (start 137.8328 101.0028) (end 138.43 101.6) (width 0.2) (layer "B.Cu") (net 7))
 (segment (start 137.8328 85.9428) (end 137.8328 101.0028) (width 0.2) (layer "B.Cu") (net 7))
 (segment (start 141.4555 78.7298) (end 163.83 78.7298) (width 0.2) (layer "F.Cu") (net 12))
 (segment (start 138.9257 76.2) (end 141.4555 78.7298) (width 0.2) (layer "F.Cu") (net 12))
 (segment (start 126.22 76.2) (end 138.9257 76.2) (width 0.2) (layer "F.Cu") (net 12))
 (via (at 163.83 78.7298) (size 0.6) (drill 0.3) (layers "F.Cu" "B.Cu") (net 12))
 (segment (start 163.83 101.6) (end 163.83 78.7298) (width 0.2) (layer "B.Cu") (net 12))
 (segment (start 124.9836 79.9764) (end 112.0356 79.9764) (width 0.2) (layer "F.Cu") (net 4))
 (segment (start 126.22 78.74) (end 124.9836 79.9764) (width 0.2) (layer "F.Cu") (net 4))
 (via (at 112.0356 79.9764) (size 0.6) (drill 0.3) (layers "F.Cu" "B.Cu") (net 4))
 (segment (start 110.3474 121.7774) (end 110.3474 81.6646) (width 0.2) (layer "B.Cu") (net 4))
 (segment (start 113.03 124.46) (end 110.3474 121.7774) (width 0.2) (layer "B.Cu") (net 4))
 (segment (start 110.3474 81.6646) (end 112.0356 79.9764) (width 0.2) (layer "B.Cu") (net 4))
 (segment (start 131.9558 82.1892) (end 127.1292 82.1892) (width 0.2) (layer "F.Cu") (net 2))
 (segment (start 127.1292 82.1892) (end 126.22 81.28) (width 0.2) (layer "F.Cu") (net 2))
 (via (at 131.9558 82.1892) (size 0.6) (drill 0.3) (layers "F.Cu" "B.Cu") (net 2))
 (segment (start 131.9558 117.9858) (end 131.9558 82.1892) (width 0.2) (layer "B.Cu") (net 2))
 (segment (start 138.43 124.46) (end 131.9558 117.9858) (width 0.2) (layer "B.Cu") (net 2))
 (segment (start 114.6145 123.3845) (end 113.9631 122.7331) (width 0.2) (layer "F.Cu") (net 3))
 (segment (start 111.2325 76.2706) (end 109.2906 76.2706) (width 0.2) (layer "F.Cu") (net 3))
 (segment (start 144.78 124.46) (end 143.3526 123.0326) (width 0.2) (layer "F.Cu") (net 3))
 (segment (start 163.83 124.46) (end 144.78 124.46) (width 0.2) (layer "F.Cu") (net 3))
 (segment (start 109.2906 76.2706) (end 109.22 76.2) (width 0.2) (layer "F.Cu") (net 3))
 (segment (start 113.9631 122.7331) (end 109.92 122.7331) (width 0.2) (layer "F.Cu") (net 3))
 (segment (start 120.4555 123.3845) (end 114.6145 123.3845) (width 0.2) (layer "F.Cu") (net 3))
 (segment (start 143.3526 123.0326) (end 120.8074 123.0326) (width 0.2) (layer "F.Cu") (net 3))
 (segment (start 120.8074 123.0326) (end 120.4555 123.3845) (width 0.2) (layer "F.Cu") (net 3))
 (via (at 111.2325 76.2706) (size 0.6) (drill 0.3) (layers "F.Cu" "B.Cu") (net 3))
 (via (at 109.92 122.7331) (size 0.6) (drill 0.3) (layers "F.Cu" "B.Cu") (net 3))
 (segment (start 109.92 77.5831) (end 109.92 122.7331) (width 0.2) (layer "B.Cu") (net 3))
 (segment (start 111.2325 76.2706) (end 109.92 77.5831) (width 0.2) (layer "B.Cu") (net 3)))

